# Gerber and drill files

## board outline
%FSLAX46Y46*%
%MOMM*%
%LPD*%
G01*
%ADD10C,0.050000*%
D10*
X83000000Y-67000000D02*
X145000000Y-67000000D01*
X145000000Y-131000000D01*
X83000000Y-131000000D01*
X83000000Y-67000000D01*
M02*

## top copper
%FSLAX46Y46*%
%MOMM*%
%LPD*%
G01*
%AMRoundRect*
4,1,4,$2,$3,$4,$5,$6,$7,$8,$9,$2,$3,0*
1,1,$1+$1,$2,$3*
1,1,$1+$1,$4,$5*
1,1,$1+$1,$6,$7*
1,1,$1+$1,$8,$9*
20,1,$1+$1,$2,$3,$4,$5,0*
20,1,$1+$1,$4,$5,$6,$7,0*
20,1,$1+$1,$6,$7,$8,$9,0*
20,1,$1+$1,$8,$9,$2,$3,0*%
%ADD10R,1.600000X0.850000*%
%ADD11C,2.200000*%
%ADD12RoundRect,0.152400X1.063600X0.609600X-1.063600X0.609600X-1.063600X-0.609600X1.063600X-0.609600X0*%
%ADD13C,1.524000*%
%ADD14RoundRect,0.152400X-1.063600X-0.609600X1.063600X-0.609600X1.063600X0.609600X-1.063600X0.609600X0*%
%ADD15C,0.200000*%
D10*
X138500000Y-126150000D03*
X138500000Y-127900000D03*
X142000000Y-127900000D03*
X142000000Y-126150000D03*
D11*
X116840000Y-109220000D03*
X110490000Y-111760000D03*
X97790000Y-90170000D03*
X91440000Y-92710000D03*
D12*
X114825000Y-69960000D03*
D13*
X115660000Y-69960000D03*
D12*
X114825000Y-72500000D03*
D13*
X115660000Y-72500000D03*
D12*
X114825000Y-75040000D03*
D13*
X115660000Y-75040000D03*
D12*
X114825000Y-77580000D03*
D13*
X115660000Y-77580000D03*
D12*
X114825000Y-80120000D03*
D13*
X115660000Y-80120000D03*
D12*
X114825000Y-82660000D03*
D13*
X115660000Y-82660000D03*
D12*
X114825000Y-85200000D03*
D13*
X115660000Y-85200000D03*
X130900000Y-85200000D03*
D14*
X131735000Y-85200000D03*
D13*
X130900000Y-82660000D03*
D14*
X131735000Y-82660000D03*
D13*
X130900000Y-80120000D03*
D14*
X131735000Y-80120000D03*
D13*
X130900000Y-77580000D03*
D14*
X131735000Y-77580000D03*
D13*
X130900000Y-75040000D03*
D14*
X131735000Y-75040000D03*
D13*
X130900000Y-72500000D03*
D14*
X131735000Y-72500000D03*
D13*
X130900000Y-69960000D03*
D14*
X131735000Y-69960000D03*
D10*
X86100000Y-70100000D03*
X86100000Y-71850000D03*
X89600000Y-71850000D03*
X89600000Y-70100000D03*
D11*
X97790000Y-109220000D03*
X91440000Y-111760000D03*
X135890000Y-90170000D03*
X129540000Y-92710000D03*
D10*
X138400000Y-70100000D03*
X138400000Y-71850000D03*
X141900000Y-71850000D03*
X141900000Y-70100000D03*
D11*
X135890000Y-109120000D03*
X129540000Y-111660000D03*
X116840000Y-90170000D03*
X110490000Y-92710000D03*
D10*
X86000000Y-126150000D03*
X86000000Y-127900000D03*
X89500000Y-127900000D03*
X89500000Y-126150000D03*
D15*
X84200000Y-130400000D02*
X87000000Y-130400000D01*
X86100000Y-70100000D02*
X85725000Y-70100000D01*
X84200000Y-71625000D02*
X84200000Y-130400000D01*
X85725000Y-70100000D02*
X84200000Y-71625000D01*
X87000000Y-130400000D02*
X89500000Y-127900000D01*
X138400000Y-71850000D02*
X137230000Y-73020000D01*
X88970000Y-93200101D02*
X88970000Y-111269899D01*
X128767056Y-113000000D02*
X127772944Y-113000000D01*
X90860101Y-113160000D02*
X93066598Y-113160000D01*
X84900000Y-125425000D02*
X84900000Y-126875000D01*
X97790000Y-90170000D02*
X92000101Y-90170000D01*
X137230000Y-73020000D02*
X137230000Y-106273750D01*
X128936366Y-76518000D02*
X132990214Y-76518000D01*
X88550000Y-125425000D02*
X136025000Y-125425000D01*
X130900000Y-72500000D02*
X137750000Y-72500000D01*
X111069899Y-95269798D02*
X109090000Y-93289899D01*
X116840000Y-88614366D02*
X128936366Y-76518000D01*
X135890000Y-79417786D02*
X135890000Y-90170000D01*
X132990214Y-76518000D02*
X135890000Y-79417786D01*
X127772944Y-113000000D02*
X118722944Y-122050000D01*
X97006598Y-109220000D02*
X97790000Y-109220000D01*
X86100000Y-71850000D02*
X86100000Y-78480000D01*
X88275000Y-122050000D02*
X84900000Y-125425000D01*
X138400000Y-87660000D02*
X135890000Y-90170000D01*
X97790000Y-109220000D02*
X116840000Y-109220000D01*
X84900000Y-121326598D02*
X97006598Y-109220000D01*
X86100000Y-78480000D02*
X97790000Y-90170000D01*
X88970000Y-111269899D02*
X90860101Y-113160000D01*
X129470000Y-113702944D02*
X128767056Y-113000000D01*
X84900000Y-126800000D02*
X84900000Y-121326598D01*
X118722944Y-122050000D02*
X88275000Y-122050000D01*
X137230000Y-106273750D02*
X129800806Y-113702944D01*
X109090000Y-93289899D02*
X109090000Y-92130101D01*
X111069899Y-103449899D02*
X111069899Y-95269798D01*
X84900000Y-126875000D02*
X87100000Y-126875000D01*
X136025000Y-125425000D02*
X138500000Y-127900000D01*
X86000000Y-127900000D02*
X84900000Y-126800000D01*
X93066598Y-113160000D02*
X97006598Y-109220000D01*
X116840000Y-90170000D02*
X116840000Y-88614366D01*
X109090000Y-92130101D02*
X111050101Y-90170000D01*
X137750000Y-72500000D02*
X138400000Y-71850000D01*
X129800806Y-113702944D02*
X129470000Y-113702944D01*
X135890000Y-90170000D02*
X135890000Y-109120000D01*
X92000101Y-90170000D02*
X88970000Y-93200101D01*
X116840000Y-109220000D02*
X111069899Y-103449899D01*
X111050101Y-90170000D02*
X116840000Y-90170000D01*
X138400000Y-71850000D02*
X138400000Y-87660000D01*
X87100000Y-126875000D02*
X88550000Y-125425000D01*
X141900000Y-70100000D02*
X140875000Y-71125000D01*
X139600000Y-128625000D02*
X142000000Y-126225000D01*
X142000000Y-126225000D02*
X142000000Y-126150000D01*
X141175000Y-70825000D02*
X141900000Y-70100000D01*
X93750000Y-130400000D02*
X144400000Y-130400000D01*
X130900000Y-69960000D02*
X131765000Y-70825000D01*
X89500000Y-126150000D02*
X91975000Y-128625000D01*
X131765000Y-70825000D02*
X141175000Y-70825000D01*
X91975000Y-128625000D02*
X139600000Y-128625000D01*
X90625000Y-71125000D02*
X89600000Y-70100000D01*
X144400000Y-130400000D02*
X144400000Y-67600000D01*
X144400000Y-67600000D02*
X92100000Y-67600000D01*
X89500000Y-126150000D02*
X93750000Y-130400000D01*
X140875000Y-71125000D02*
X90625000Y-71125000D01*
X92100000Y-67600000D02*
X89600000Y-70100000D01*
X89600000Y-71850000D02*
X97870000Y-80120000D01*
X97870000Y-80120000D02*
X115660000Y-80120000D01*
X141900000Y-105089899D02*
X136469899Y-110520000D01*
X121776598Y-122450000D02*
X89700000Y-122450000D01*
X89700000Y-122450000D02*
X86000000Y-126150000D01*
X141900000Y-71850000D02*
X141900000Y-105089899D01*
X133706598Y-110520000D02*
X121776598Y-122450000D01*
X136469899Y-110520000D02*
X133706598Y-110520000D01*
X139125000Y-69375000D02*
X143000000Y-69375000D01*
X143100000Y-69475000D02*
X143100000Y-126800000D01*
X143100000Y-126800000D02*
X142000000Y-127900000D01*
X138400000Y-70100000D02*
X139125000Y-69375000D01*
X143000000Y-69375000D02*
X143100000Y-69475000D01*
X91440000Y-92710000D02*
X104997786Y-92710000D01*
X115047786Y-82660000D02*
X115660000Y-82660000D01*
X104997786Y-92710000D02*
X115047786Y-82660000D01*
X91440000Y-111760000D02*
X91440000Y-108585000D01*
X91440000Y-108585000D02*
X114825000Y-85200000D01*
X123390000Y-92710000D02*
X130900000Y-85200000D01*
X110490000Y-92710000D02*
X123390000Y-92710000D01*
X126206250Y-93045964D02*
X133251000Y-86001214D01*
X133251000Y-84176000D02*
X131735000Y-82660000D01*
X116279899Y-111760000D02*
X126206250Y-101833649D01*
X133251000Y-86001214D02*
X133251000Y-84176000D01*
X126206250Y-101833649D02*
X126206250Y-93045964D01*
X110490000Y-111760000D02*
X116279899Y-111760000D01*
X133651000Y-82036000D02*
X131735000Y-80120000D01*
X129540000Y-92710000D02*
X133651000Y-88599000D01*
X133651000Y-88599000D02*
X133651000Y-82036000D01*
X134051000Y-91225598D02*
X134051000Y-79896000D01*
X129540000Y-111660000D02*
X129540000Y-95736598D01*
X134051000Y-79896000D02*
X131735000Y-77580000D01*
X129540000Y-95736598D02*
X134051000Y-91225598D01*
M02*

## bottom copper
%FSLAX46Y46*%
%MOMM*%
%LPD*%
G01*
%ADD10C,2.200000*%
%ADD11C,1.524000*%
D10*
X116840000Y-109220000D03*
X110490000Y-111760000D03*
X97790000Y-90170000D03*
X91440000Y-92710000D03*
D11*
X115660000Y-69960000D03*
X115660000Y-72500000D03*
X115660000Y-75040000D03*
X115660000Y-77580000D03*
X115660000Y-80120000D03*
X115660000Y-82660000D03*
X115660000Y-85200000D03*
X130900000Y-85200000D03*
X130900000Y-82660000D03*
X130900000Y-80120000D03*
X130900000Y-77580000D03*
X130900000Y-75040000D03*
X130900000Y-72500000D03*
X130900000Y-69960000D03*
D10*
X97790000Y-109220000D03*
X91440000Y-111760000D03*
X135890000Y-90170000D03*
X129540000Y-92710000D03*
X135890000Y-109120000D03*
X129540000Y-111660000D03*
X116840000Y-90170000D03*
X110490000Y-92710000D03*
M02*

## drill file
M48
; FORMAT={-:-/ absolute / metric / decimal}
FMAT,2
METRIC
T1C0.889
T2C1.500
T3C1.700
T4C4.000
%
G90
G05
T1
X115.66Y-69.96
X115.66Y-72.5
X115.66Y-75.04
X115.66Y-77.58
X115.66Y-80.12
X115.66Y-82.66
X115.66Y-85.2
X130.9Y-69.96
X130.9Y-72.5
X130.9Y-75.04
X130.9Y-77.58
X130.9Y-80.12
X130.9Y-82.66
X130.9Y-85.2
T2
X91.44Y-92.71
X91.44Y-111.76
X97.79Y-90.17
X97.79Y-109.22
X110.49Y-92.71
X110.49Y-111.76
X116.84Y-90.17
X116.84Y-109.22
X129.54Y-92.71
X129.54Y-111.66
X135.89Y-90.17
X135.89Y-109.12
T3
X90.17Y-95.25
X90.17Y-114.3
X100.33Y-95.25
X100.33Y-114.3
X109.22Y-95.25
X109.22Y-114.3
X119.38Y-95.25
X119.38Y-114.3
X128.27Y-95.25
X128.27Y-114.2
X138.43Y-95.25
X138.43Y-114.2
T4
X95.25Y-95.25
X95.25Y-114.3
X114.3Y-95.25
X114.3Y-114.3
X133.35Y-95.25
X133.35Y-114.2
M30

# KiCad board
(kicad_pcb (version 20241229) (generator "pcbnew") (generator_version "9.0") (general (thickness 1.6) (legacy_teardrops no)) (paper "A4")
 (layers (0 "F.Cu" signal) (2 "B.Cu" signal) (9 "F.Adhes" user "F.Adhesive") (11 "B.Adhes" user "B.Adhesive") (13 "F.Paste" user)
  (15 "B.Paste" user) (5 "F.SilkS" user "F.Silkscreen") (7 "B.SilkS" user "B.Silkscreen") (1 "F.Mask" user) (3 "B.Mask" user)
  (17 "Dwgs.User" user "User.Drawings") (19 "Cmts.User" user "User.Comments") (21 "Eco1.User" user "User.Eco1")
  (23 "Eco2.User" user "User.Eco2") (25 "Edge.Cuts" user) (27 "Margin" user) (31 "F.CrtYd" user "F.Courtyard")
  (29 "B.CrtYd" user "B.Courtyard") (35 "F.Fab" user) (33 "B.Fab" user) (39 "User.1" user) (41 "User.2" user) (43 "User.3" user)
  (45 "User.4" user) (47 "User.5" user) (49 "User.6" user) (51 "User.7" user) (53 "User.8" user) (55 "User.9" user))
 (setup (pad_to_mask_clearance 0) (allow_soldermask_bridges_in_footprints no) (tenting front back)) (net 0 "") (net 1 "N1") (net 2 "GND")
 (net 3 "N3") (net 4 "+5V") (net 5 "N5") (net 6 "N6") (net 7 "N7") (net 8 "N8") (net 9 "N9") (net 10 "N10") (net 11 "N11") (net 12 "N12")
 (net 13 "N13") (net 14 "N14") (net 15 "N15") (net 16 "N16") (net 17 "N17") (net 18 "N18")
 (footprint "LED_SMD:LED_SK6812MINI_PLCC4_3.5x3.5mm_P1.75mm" (layer "F.Cu") (at 140.25 127.025)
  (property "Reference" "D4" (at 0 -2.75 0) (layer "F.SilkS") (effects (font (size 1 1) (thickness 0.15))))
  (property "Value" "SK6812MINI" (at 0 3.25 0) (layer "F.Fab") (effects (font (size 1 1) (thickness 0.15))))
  (pad "1" smd rect (at -1.75 -0.875) (size 1.6 0.85) (layers "F.Cu" "F.Mask" "F.Paste") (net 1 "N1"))
  (pad "2" smd rect (at -1.75 0.875) (size 1.6 0.85) (layers "F.Cu" "F.Mask" "F.Paste") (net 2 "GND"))
  (pad "3" smd rect (at 1.75 0.875) (size 1.6 0.85) (layers "F.Cu" "F.Mask" "F.Paste") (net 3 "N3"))
  (pad "4" smd rect (at 1.75 -0.875) (size 1.6 0.85) (layers "F.Cu" "F.Mask" "F.Paste") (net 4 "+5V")))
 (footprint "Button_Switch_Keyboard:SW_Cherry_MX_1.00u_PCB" (layer "F.Cu") (at 116.84 109.22)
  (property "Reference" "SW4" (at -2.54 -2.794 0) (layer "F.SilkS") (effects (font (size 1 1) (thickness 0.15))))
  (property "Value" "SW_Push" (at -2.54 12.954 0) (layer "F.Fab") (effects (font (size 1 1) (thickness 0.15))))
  (pad "" np_thru_hole circle (at -7.62 5.08) (size 1.7 1.7) (drill 1.7) (layers "*.Cu" "*.Mask"))
  (pad "" np_thru_hole circle (at -2.54 5.08) (size 4 4) (drill 4) (layers "*.Cu" "*.Mask"))
  (pad "" np_thru_hole circle (at 2.54 5.08) (size 1.7 1.7) (drill 1.7) (layers "*.Cu" "*.Mask"))
  (pad "1" thru_hole circle (at 0 0) (size 2.2 2.2) (drill 1.5) (layers "*.Cu" "*.Mask") (remove_unused_layers no) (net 2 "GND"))
  (pad "2" thru_hole circle (at -6.35 2.54) (size 2.2 2.2) (drill 1.5) (layers "*.Cu" "*.Mask") (remove_unused_layers no) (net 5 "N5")))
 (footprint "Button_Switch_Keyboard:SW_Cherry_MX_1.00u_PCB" (layer "F.Cu") (at 97.79 90.17)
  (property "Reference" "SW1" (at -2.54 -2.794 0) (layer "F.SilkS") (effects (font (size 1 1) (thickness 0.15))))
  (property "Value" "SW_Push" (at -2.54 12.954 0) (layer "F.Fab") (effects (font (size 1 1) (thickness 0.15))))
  (pad "" np_thru_hole circle (at -7.62 5.08) (size 1.7 1.7) (drill 1.7) (layers "*.Cu" "*.Mask"))
  (pad "" np_thru_hole circle (at -2.54 5.08) (size 4 4) (drill 4) (layers "*.Cu" "*.Mask"))
  (pad "" np_thru_hole circle (at 2.54 5.08) (size 1.7 1.7) (drill 1.7) (layers "*.Cu" "*.Mask"))
  (pad "1" thru_hole circle (at 0 0) (size 2.2 2.2) (drill 1.5) (layers "*.Cu" "*.Mask") (remove_unused_layers no) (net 2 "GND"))
  (pad "2" thru_hole circle (at -6.35 2.54) (size 2.2 2.2) (drill 1.5) (layers "*.Cu" "*.Mask") (remove_unused_layers no) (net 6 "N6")))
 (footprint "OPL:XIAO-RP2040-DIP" (layer "F.Cu") (at 123.28 77.58)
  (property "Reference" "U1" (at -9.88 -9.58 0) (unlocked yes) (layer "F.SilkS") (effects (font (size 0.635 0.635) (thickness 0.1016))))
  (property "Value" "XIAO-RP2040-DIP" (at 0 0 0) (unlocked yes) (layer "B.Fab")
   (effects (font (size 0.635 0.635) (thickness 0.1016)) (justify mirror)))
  (pad "1" smd roundrect (at -8.455 -7.62 180) (size 2.432 1.524) (layers "F.Cu" "F.Mask") (roundrect_rratio 0.1) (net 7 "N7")
   (thermal_bridge_angle 45))
  (pad "1" thru_hole circle (at -7.62 -7.62 180) (size 1.524 1.524) (drill 0.889) (layers "*.Cu" "*.Mask") (remove_unused_layers no)
   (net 7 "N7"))
  (pad "2" smd roundrect (at -8.455 -5.08 180) (size 2.432 1.524) (layers "F.Cu" "F.Mask") (roundrect_rratio 0.1) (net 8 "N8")
   (thermal_bridge_angle 45))
  (pad "2" thru_hole circle (at -7.62 -5.08 180) (size 1.524 1.524) (drill 0.889) (layers "*.Cu" "*.Mask") (remove_unused_layers no)
   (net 8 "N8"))
  (pad "3" smd roundrect (at -8.455 -2.54 180) (size 2.432 1.524) (layers "F.Cu" "F.Mask") (roundrect_rratio 0.1) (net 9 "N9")
   (thermal_bridge_angle 45))
  (pad "3" thru_hole circle (at -7.62 -2.54 180) (size 1.524 1.524) (drill 0.889) (layers "*.Cu" "*.Mask") (remove_unused_layers no)
   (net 9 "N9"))
  (pad "4" smd roundrect (at -8.455 0 180) (size 2.432 1.524) (layers "F.Cu" "F.Mask") (roundrect_rratio 0.1) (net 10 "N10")
   (thermal_bridge_angle 45))
  (pad "4" thru_hole circle (at -7.62 0 180) (size 1.524 1.524) (drill 0.889) (layers "*.Cu" "*.Mask") (remove_unused_layers no)
   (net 10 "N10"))
  (pad "5" smd roundrect (at -8.455 2.54 180) (size 2.432 1.524) (layers "F.Cu" "F.Mask") (roundrect_rratio 0.1) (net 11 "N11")
   (thermal_bridge_angle 45))
  (pad "5" thru_hole circle (at -7.62 2.54 180) (size 1.524 1.524) (drill 0.889) (layers "*.Cu" "*.Mask") (remove_unused_layers no)
   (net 11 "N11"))
  (pad "6" smd roundrect (at -8.455 5.08 180) (size 2.432 1.524) (layers "F.Cu" "F.Mask") (roundrect_rratio 0.1) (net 6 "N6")
   (thermal_bridge_angle 45))
  (pad "6" thru_hole circle (at -7.62 5.08 180) (size 1.524 1.524) (drill 0.889) (layers "*.Cu" "*.Mask") (remove_unused_layers no)
   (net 6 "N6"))
  (pad "7" smd roundrect (at -8.455 7.62 180) (size 2.432 1.524) (layers "F.Cu" "F.Mask") (roundrect_rratio 0.1) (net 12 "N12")
   (thermal_bridge_angle 45))
  (pad "7" thru_hole circle (at -7.62 7.62 180) (size 1.524 1.524) (drill 0.889) (layers "*.Cu" "*.Mask") (remove_unused_layers no)
   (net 12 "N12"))
  (pad "8" thru_hole circle (at 7.62 7.62) (size 1.524 1.524) (drill 0.889) (layers "*.Cu" "*.Mask") (remove_unused_layers no)
   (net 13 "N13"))
  (pad "8" smd roundrect (at 8.455 7.62) (size 2.432 1.524) (layers "F.Cu" "F.Mask") (roundrect_rratio 0.1) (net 13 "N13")
   (thermal_bridge_angle 45))
  (pad "9" thru_hole circle (at 7.62 5.08) (size 1.524 1.524) (drill 0.889) (layers "*.Cu" "*.Mask") (remove_unused_layers no) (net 5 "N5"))
  (pad "9" smd roundrect (at 8.455 5.08) (size 2.432 1.524) (layers "F.Cu" "F.Mask") (roundrect_rratio 0.1) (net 5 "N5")
   (thermal_bridge_angle 45))
  (pad "10" thru_hole circle (at 7.62 2.54) (size 1.524 1.524) (drill 0.889) (layers "*.Cu" "*.Mask") (remove_unused_layers no)
   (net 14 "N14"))
  (pad "10" smd roundrect (at 8.455 2.54) (size 2.432 1.524) (layers "F.Cu" "F.Mask") (roundrect_rratio 0.1) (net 14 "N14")
   (thermal_bridge_angle 45))
  (pad "11" thru_hole circle (at 7.62 0) (size 1.524 1.524) (drill 0.889) (layers "*.Cu" "*.Mask") (remove_unused_layers no) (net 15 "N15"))
  (pad "11" smd roundrect (at 8.455 0) (size 2.432 1.524) (layers "F.Cu" "F.Mask") (roundrect_rratio 0.1) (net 15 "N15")
   (thermal_bridge_angle 45))
  (pad "12" thru_hole circle (at 7.62 -2.54) (size 1.524 1.524) (drill 0.889) (layers "*.Cu" "*.Mask") (remove_unused_layers no)
   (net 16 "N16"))
  (pad "12" smd roundrect (at 8.455 -2.54) (size 2.432 1.524) (layers "F.Cu" "F.Mask") (roundrect_rratio 0.1) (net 16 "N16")
   (thermal_bridge_angle 45))
  (pad "13" thru_hole circle (at 7.62 -5.08) (size 1.524 1.524) (drill 0.889) (layers "*.Cu" "*.Mask") (remove_unused_layers no)
   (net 2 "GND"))
  (pad "13" smd roundrect (at 8.455 -5.08) (size 2.432 1.524) (layers "F.Cu" "F.Mask") (roundrect_rratio 0.1) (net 2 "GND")
   (thermal_bridge_angle 45))
  (pad "14" thru_hole circle (at 7.62 -7.62) (size 1.524 1.524) (drill 0.889) (layers "*.Cu" "*.Mask") (remove_unused_layers no)
   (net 4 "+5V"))
  (pad "14" smd roundrect (at 8.455 -7.62) (size 2.432 1.524) (layers "F.Cu" "F.Mask") (roundrect_rratio 0.1) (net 4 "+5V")
   (thermal_bridge_angle 45)))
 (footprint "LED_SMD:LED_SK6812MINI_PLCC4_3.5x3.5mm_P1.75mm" (layer "F.Cu") (at 87.85 70.975)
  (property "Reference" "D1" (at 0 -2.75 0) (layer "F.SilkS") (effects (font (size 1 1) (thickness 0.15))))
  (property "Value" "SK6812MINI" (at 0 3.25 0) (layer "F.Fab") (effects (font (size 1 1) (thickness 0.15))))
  (pad "1" smd rect (at -1.75 -0.875) (size 1.6 0.85) (layers "F.Cu" "F.Mask" "F.Paste") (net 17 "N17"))
  (pad "2" smd rect (at -1.75 0.875) (size 1.6 0.85) (layers "F.Cu" "F.Mask" "F.Paste") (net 2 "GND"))
  (pad "3" smd rect (at 1.75 0.875) (size 1.6 0.85) (layers "F.Cu" "F.Mask" "F.Paste") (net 11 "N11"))
  (pad "4" smd rect (at 1.75 -0.875) (size 1.6 0.85) (layers "F.Cu" "F.Mask" "F.Paste") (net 4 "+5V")))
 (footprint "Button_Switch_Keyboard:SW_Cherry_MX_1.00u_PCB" (layer "F.Cu") (at 97.79 109.22)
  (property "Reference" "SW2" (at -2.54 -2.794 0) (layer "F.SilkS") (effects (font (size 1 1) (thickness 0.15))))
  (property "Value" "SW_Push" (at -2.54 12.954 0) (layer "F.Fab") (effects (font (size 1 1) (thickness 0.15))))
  (pad "" np_thru_hole circle (at -7.62 5.08) (size 1.7 1.7) (drill 1.7) (layers "*.Cu" "*.Mask"))
  (pad "" np_thru_hole circle (at -2.54 5.08) (size 4 4) (drill 4) (layers "*.Cu" "*.Mask"))
  (pad "" np_thru_hole circle (at 2.54 5.08) (size 1.7 1.7) (drill 1.7) (layers "*.Cu" "*.Mask"))
  (pad "1" thru_hole circle (at 0 0) (size 2.2 2.2) (drill 1.5) (layers "*.Cu" "*.Mask") (remove_unused_layers no) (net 2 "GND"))
  (pad "2" thru_hole circle (at -6.35 2.54) (size 2.2 2.2) (drill 1.5) (layers "*.Cu" "*.Mask") (remove_unused_layers no) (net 12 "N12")))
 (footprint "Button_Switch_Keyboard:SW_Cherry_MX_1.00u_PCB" (layer "F.Cu") (at 135.89 90.17)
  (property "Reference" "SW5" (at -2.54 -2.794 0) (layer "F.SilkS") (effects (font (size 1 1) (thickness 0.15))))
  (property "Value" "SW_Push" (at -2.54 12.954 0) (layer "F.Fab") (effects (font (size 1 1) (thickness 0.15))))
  (pad "" np_thru_hole circle (at -7.62 5.08) (size 1.7 1.7) (drill 1.7) (layers "*.Cu" "*.Mask"))
  (pad "" np_thru_hole circle (at -2.54 5.08) (size 4 4) (drill 4) (layers "*.Cu" "*.Mask"))
  (pad "" np_thru_hole circle (at 2.54 5.08) (size 1.7 1.7) (drill 1.7) (layers "*.Cu" "*.Mask"))
  (pad "1" thru_hole circle (at 0 0) (size 2.2 2.2) (drill 1.5) (layers "*.Cu" "*.Mask") (remove_unused_layers no) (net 2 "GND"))
  (pad "2" thru_hole circle (at -6.35 2.54) (size 2.2 2.2) (drill 1.5) (layers "*.Cu" "*.Mask") (remove_unused_layers no) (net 14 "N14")))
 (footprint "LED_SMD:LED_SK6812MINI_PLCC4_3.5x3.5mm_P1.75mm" (layer "F.Cu") (at 140.15 70.975)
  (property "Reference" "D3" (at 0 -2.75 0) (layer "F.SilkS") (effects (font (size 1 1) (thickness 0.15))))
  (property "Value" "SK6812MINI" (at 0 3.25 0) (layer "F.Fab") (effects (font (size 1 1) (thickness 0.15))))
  (pad "1" smd rect (at -1.75 -0.875) (size 1.6 0.85) (layers "F.Cu" "F.Mask" "F.Paste") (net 3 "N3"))
  (pad "2" smd rect (at -1.75 0.875) (size 1.6 0.85) (layers "F.Cu" "F.Mask" "F.Paste") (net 2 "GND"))
  (pad "3" smd rect (at 1.75 0.875) (size 1.6 0.85) (layers "F.Cu" "F.Mask" "F.Paste") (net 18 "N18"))
  (pad "4" smd rect (at 1.75 -0.875) (size 1.6 0.85) (layers "F.Cu" "F.Mask" "F.Paste") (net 4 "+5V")))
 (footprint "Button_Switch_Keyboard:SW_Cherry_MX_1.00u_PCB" (layer "F.Cu") (at 135.89 109.12)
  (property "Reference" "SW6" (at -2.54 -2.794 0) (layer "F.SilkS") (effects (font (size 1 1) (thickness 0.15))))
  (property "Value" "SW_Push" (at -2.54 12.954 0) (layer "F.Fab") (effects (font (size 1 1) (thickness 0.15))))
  (pad "" np_thru_hole circle (at -7.62 5.08) (size 1.7 1.7) (drill 1.7) (layers "*.Cu" "*.Mask"))
  (pad "" np_thru_hole circle (at -2.54 5.08) (size 4 4) (drill 4) (layers "*.Cu" "*.Mask"))
  (pad "" np_thru_hole circle (at 2.54 5.08) (size 1.7 1.7) (drill 1.7) (layers "*.Cu" "*.Mask"))
  (pad "1" thru_hole circle (at 0 0) (size 2.2 2.2) (drill 1.5) (layers "*.Cu" "*.Mask") (remove_unused_layers no) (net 2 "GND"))
  (pad "2" thru_hole circle (at -6.35 2.54) (size 2.2 2.2) (drill 1.5) (layers "*.Cu" "*.Mask") (remove_unused_layers no) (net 15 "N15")))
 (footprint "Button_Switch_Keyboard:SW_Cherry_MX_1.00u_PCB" (layer "F.Cu") (at 116.84 90.17)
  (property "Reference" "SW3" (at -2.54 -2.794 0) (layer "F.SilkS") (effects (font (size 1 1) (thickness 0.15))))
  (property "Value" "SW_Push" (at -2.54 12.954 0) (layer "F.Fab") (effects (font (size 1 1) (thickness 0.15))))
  (pad "" np_thru_hole circle (at -7.62 5.08) (size 1.7 1.7) (drill 1.7) (layers "*.Cu" "*.Mask"))
  (pad "" np_thru_hole circle (at -2.54 5.08) (size 4 4) (drill 4) (layers "*.Cu" "*.Mask"))
  (pad "" np_thru_hole circle (at 2.54 5.08) (size 1.7 1.7) (drill 1.7) (layers "*.Cu" "*.Mask"))
  (pad "1" thru_hole circle (at 0 0) (size 2.2 2.2) (drill 1.5) (layers "*.Cu" "*.Mask") (remove_unused_layers no) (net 2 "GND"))
  (pad "2" thru_hole circle (at -6.35 2.54) (size 2.2 2.2) (drill 1.5) (layers "*.Cu" "*.Mask") (remove_unused_layers no) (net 13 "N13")))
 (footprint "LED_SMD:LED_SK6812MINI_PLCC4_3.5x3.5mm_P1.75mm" (layer "F.Cu") (at 87.75 127.025)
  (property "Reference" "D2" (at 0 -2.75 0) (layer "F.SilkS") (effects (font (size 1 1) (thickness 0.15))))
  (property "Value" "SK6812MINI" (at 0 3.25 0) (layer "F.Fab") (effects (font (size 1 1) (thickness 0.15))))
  (pad "1" smd rect (at -1.75 -0.875) (size 1.6 0.85) (layers "F.Cu" "F.Mask" "F.Paste") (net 18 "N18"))
  (pad "2" smd rect (at -1.75 0.875) (size 1.6 0.85) (layers "F.Cu" "F.Mask" "F.Paste") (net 2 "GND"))
  (pad "3" smd rect (at 1.75 0.875) (size 1.6 0.85) (layers "F.Cu" "F.Mask" "F.Paste") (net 17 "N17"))
  (pad "4" smd rect (at 1.75 -0.875) (size 1.6 0.85) (layers "F.Cu" "F.Mask" "F.Paste") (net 4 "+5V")))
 (gr_rect (start 83 67) (end 145 131) (stroke (width 0.05) (type default)) (fill no) (layer "Edge.Cuts"))
 (segment (start 84.2 130.4) (end 87 130.4) (width 0.2) (layer "F.Cu") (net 17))
 (segment (start 86.1 70.1) (end 85.725 70.1) (width 0.2) (layer "F.Cu") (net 17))
 (segment (start 84.2 71.625) (end 84.2 130.4) (width 0.2) (layer "F.Cu") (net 17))
 (segment (start 85.725 70.1) (end 84.2 71.625) (width 0.2) (layer "F.Cu") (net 17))
 (segment (start 87 130.4) (end 89.5 127.9) (width 0.2) (layer "F.Cu") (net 17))
 (segment (start 138.4 71.85) (end 137.23 73.02) (width 0.2) (layer "F.Cu") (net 2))
 (segment (start 88.97 93.200101) (end 88.97 111.269899) (width 0.2) (layer "F.Cu") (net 2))
 (segment (start 128.767056 113) (end 127.772944 113) (width 0.2) (layer "F.Cu") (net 2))
 (segment (start 90.860101 113.16) (end 93.066598 113.16) (width 0.2) (layer "F.Cu") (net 2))
 (segment (start 84.9 125.425) (end 84.9 126.875) (width 0.2) (layer "F.Cu") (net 2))
 (segment (start 97.79 90.17) (end 92.000101 90.17) (width 0.2) (layer "F.Cu") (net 2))
 (segment (start 137.23 73.02) (end 137.23 106.27375) (width 0.2) (layer "F.Cu") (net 2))
 (segment (start 128.936366 76.518) (end 132.990214 76.518) (width 0.2) (layer "F.Cu") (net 2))
 (segment (start 88.55 125.425) (end 136.025 125.425) (width 0.2) (layer "F.Cu") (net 2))
 (segment (start 130.9 72.5) (end 137.75 72.5) (width 0.2) (layer "F.Cu") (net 2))
 (segment (start 111.069899 95.269798) (end 109.09 93.289899) (width 0.2) (layer "F.Cu") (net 2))
 (segment (start 116.84 88.614366) (end 128.936366 76.518) (width 0.2) (layer "F.Cu") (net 2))
 (segment (start 135.89 79.417786) (end 135.89 90.17) (width 0.2) (layer "F.Cu") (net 2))
 (segment (start 132.990214 76.518) (end 135.89 79.417786) (width 0.2) (layer "F.Cu") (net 2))
 (segment (start 127.772944 113) (end 118.722944 122.05) (width 0.2) (layer "F.Cu") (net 2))
 (segment (start 97.006598 109.22) (end 97.79 109.22) (width 0.2) (layer "F.Cu") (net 2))
 (segment (start 86.1 71.85) (end 86.1 78.48) (width 0.2) (layer "F.Cu") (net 2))
 (segment (start 88.275 122.05) (end 84.9 125.425) (width 0.2) (layer "F.Cu") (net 2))
 (segment (start 138.4 87.66) (end 135.89 90.17) (width 0.2) (layer "F.Cu") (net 2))
 (segment (start 97.79 109.22) (end 116.84 109.22) (width 0.2) (layer "F.Cu") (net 2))
 (segment (start 84.9 121.326598) (end 97.006598 109.22) (width 0.2) (layer "F.Cu") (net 2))
 (segment (start 86.1 78.48) (end 97.79 90.17) (width 0.2) (layer "F.Cu") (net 2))
 (segment (start 88.97 111.269899) (end 90.860101 113.16) (width 0.2) (layer "F.Cu") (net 2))
 (segment (start 129.47 113.702944) (end 128.767056 113) (width 0.2) (layer "F.Cu") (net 2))
 (segment (start 84.9 126.8) (end 84.9 121.326598) (width 0.2) (layer "F.Cu") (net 2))
 (segment (start 118.722944 122.05) (end 88.275 122.05) (width 0.2) (layer "F.Cu") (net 2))
 (segment (start 137.23 106.27375) (end 129.800806 113.702944) (width 0.2) (layer "F.Cu") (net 2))
 (segment (start 109.09 93.289899) (end 109.09 92.130101) (width 0.2) (layer "F.Cu") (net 2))
 (segment (start 111.069899 103.449899) (end 111.069899 95.269798) (width 0.2) (layer "F.Cu") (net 2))
 (segment (start 84.9 126.875) (end 87.1 126.875) (width 0.2) (layer "F.Cu") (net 2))
 (segment (start 136.025 125.425) (end 138.5 127.9) (width 0.2) (layer "F.Cu") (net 2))
 (segment (start 86 127.9) (end 84.9 126.8) (width 0.2) (layer "F.Cu") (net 2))
 (segment (start 93.066598 113.16) (end 97.006598 109.22) (width 0.2) (layer "F.Cu") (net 2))
 (segment (start 116.84 90.17) (end 116.84 88.614366) (width 0.2) (layer "F.Cu") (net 2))
 (segment (start 109.09 92.130101) (end 111.050101 90.17) (width 0.2) (layer "F.Cu") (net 2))
 (segment (start 137.75 72.5) (end 138.4 71.85) (width 0.2) (layer "F.Cu") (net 2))
 (segment (start 129.800806 113.702944) (end 129.47 113.702944) (width 0.2) (layer "F.Cu") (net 2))
 (segment (start 135.89 90.17) (end 135.89 109.12) (width 0.2) (layer "F.Cu") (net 2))
 (segment (start 92.000101 90.17) (end 88.97 93.200101) (width 0.2) (layer "F.Cu") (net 2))
 (segment (start 116.84 109.22) (end 111.069899 103.449899) (width 0.2) (layer "F.Cu") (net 2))
 (segment (start 111.050101 90.17) (end 116.84 90.17) (width 0.2) (layer "F.Cu") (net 2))
 (segment (start 138.4 71.85) (end 138.4 87.66) (width 0.2) (layer "F.Cu") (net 2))
 (segment (start 87.1 126.875) (end 88.55 125.425) (width 0.2) (layer "F.Cu") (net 2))
 (segment (start 141.9 70.1) (end 140.875 71.125) (width 0.2) (layer "F.Cu") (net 4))
 (segment (start 139.6 128.625) (end 142 126.225) (width 0.2) (layer "F.Cu") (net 4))
 (segment (start 142 126.225) (end 142 126.15) (width 0.2) (layer "F.Cu") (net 4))
 (segment (start 141.175 70.825) (end 141.9 70.1) (width 0.2) (layer "F.Cu") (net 4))
 (segment (start 93.75 130.4) (end 144.4 130.4) (width 0.2) (layer "F.Cu") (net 4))
 (segment (start 130.9 69.96) (end 131.765 70.825) (width 0.2) (layer "F.Cu") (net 4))
 (segment (start 89.5 126.15) (end 91.975 128.625) (width 0.2) (layer "F.Cu") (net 4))
 (segment (start 131.765 70.825) (end 141.175 70.825) (width 0.2) (layer "F.Cu") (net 4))
 (segment (start 91.975 128.625) (end 139.6 128.625) (width 0.2) (layer "F.Cu") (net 4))
 (segment (start 90.625 71.125) (end 89.6 70.1) (width 0.2) (layer "F.Cu") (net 4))
 (segment (start 144.4 130.4) (end 144.4 67.6) (width 0.2) (layer "F.Cu") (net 4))
 (segment (start 144.4 67.6) (end 92.1 67.6) (width 0.2) (layer "F.Cu") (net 4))
 (segment (start 89.5 126.15) (end 93.75 130.4) (width 0.2) (layer "F.Cu") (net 4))
 (segment (start 140.875 71.125) (end 90.625 71.125) (width 0.2) (layer "F.Cu") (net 4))
 (segment (start 92.1 67.6) (end 89.6 70.1) (width 0.2) (layer "F.Cu") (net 4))
 (segment (start 89.6 71.85) (end 97.87 80.12) (width 0.2) (layer "F.Cu") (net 11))
 (segment (start 97.87 80.12) (end 115.66 80.12) (width 0.2) (layer "F.Cu") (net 11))
 (segment (start 141.9 105.089899) (end 136.469899 110.52) (width 0.2) (layer "F.Cu") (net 18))
 (segment (start 121.776598 122.45) (end 89.7 122.45) (width 0.2) (layer "F.Cu") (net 18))
 (segment (start 89.7 122.45) (end 86 126.15) (width 0.2) (layer "F.Cu") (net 18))
 (segment (start 141.9 71.85) (end 141.9 105.089899) (width 0.2) (layer "F.Cu") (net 18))
 (segment (start 133.706598 110.52) (end 121.776598 122.45) (width 0.2) (layer "F.Cu") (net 18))
 (segment (start 136.469899 110.52) (end 133.706598 110.52) (width 0.2) (layer "F.Cu") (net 18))
 (segment (start 139.125 69.375) (end 143 69.375) (width 0.2) (layer "F.Cu") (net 3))
 (segment (start 143.1 69.475) (end 143.1 126.8) (width 0.2) (layer "F.Cu") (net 3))
 (segment (start 143.1 126.8) (end 142 127.9) (width 0.2) (layer "F.Cu") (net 3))
 (segment (start 138.4 70.1) (end 139.125 69.375) (width 0.2) (layer "F.Cu") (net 3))
 (segment (start 143 69.375) (end 143.1 69.475) (width 0.2) (layer "F.Cu") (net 3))
 (segment (start 91.44 92.71) (end 104.997786 92.71) (width 0.2) (layer "F.Cu") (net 6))
 (segment (start 115.047786 82.66) (end 115.66 82.66) (width 0.2) (layer "F.Cu") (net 6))
 (segment (start 104.997786 92.71) (end 115.047786 82.66) (width 0.2) (layer "F.Cu") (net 6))
 (segment (start 91.44 111.76) (end 91.44 108.585) (width 0.2) (layer "F.Cu") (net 12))
 (segment (start 91.44 108.585) (end 114.825 85.2) (width 0.2) (layer "F.Cu") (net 12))
 (segment (start 123.39 92.71) (end 130.9 85.2) (width 0.2) (layer "F.Cu") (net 13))
 (segment (start 110.49 92.71) (end 123.39 92.71) (width 0.2) (layer "F.Cu") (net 13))
 (segment (start 126.20625 93.045964) (end 133.251 86.001214) (width 0.2) (layer "F.Cu") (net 5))
 (segment (start 133.251 84.176) (end 131.735 82.66) (width 0.2) (layer "F.Cu") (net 5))
 (segment (start 116.279899 111.76) (end 126.20625 101.833649) (width 0.2) (layer "F.Cu") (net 5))
 (segment (start 133.251 86.001214) (end 133.251 84.176) (width 0.2) (layer "F.Cu") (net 5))
 (segment (start 126.20625 101.833649) (end 126.20625 93.045964) (width 0.2) (layer "F.Cu") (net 5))
 (segment (start 110.49 111.76) (end 116.279899 111.76) (width 0.2) (layer "F.Cu") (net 5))
 (segment (start 133.651 82.036) (end 131.735 80.12) (width 0.2) (layer "F.Cu") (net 14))
 (segment (start 129.54 92.71) (end 133.651 88.599) (width 0.2) (layer "F.Cu") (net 14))
 (segment (start 133.651 88.599) (end 133.651 82.036) (width 0.2) (layer "F.Cu") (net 14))
 (segment (start 134.051 91.225598) (end 134.051 79.896) (width 0.2) (layer "F.Cu") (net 15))
 (segment (start 129.54 111.66) (end 129.54 95.736598) (width 0.2) (layer "F.Cu") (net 15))
 (segment (start 134.051 79.896) (end 131.735 77.58) (width 0.2) (layer "F.Cu") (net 15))
 (segment (start 129.54 95.736598) (end 134.051 91.225598) (width 0.2) (layer "F.Cu") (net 15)))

